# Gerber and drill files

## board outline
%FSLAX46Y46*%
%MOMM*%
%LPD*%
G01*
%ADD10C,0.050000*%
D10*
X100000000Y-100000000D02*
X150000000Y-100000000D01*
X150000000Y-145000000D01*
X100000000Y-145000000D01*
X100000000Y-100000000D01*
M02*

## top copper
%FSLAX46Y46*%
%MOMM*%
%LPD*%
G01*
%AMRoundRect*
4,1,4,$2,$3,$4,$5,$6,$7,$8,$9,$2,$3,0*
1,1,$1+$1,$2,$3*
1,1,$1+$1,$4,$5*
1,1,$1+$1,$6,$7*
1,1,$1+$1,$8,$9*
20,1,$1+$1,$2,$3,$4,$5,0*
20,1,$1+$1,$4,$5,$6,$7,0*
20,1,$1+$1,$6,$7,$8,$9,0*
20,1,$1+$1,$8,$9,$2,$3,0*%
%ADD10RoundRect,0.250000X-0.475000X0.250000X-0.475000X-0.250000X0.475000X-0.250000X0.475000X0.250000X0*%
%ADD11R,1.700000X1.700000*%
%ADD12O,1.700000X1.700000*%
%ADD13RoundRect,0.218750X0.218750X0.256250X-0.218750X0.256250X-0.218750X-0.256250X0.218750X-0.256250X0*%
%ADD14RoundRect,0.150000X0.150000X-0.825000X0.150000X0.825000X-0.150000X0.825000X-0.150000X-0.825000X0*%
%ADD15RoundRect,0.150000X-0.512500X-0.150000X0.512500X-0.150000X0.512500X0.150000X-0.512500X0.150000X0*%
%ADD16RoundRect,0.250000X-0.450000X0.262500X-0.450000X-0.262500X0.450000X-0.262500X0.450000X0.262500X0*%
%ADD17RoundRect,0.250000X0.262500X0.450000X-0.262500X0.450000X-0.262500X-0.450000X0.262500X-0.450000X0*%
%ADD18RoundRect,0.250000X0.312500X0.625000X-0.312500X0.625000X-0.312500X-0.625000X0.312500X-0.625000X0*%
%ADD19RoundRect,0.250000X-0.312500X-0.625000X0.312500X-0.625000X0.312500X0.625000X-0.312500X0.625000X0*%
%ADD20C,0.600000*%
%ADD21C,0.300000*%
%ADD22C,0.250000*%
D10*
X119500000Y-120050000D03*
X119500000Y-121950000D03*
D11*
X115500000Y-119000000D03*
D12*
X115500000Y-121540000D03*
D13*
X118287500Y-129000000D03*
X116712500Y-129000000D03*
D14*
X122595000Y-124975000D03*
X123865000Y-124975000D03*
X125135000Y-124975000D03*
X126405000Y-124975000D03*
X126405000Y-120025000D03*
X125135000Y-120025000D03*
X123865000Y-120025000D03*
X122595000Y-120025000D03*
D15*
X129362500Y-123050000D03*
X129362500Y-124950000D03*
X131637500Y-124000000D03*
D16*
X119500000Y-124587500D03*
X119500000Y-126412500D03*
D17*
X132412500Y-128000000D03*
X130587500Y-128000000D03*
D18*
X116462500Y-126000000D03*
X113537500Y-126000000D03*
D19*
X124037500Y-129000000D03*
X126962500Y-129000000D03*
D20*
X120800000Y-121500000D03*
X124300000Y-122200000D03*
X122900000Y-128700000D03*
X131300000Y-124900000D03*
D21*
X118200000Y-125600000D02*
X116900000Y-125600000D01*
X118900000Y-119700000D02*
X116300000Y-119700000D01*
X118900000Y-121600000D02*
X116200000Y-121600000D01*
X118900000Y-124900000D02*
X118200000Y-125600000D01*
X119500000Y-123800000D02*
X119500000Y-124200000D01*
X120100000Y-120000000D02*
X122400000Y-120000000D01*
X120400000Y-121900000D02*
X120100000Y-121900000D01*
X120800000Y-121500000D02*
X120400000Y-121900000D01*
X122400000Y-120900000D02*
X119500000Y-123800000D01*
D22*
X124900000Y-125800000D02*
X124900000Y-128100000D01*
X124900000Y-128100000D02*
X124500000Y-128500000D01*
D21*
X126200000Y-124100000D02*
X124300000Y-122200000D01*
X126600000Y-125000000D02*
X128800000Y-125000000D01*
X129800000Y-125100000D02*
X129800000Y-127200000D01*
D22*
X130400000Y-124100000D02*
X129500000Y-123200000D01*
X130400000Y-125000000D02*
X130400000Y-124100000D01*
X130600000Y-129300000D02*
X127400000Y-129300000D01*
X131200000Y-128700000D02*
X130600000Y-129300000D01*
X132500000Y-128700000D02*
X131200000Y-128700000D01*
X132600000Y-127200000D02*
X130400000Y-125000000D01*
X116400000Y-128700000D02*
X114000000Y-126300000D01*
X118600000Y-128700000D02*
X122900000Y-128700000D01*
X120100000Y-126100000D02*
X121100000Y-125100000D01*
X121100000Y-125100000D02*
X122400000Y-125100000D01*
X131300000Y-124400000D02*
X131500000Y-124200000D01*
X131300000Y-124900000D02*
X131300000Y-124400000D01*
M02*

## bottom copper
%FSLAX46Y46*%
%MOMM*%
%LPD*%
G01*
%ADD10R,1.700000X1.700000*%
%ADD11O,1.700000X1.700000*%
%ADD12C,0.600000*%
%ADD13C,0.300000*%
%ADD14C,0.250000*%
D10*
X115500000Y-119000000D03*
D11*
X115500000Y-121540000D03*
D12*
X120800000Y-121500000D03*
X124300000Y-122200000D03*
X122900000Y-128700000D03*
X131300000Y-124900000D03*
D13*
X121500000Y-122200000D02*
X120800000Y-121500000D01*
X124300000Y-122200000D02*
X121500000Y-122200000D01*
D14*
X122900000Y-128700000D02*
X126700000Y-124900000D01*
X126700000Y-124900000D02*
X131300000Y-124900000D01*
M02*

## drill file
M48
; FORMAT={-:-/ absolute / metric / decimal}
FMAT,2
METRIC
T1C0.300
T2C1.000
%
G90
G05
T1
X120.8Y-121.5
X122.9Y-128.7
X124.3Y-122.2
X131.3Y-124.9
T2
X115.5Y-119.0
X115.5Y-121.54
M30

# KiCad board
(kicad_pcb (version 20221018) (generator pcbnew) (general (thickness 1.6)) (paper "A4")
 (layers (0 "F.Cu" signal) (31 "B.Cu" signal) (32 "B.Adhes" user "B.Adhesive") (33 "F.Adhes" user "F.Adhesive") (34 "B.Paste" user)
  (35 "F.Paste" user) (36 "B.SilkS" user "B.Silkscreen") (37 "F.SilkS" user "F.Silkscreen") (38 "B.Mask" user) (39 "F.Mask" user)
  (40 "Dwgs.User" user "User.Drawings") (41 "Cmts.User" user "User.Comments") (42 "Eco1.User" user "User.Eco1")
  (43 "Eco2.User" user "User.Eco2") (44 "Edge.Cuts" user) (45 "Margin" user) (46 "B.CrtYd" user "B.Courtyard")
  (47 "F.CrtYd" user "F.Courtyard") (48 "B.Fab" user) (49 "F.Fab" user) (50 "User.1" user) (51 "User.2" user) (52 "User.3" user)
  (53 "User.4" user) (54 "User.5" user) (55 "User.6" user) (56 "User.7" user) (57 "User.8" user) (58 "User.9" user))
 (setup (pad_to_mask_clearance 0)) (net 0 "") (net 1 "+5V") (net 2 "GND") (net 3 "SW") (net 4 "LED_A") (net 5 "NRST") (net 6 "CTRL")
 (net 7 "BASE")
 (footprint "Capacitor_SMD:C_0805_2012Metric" (layer "F.Cu") (at 119.5 121 -90)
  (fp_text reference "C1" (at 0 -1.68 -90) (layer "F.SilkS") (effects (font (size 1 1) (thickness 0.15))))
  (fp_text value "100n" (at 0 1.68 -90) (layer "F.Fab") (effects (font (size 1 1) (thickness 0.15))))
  (pad "1" smd roundrect (at -0.95 0 270) (size 1 1.45) (layers "F.Cu" "F.Paste" "F.Mask") (roundrect_rratio 0.25) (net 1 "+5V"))
  (pad "2" smd roundrect (at 0.95 0 270) (size 1 1.45) (layers "F.Cu" "F.Paste" "F.Mask") (roundrect_rratio 0.25) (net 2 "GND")))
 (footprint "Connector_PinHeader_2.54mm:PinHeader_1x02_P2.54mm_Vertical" (layer "F.Cu") (at 115.5 119)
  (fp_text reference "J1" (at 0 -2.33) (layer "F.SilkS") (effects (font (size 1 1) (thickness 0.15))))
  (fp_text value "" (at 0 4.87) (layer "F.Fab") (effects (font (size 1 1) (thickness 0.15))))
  (pad "1" thru_hole rect (at 0 0) (size 1.7 1.7) (drill 1) (layers "*.Cu" "*.Mask") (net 1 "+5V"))
  (pad "2" thru_hole oval (at 0 2.54) (size 1.7 1.7) (drill 1) (layers "*.Cu" "*.Mask") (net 2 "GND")))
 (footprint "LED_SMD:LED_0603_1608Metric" (layer "F.Cu") (at 117.5 129 180)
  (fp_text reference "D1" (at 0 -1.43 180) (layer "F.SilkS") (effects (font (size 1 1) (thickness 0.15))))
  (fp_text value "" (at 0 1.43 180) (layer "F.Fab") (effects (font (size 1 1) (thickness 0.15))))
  (pad "1" smd roundrect (at -0.7875 0 180) (size 0.875 0.95) (layers "F.Cu" "F.Paste" "F.Mask") (roundrect_rratio 0.25) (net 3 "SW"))
  (pad "2" smd roundrect (at 0.7875 0 180) (size 0.875 0.95) (layers "F.Cu" "F.Paste" "F.Mask") (roundrect_rratio 0.25) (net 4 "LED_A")))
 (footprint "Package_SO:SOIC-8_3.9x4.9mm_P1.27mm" (layer "F.Cu") (at 124.5 122.5 90)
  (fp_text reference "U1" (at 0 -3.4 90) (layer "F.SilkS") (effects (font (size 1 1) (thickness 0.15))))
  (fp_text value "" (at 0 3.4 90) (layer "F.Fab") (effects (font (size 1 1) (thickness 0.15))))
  (pad "1" smd roundrect (at -2.475 -1.905 90) (size 1.95 0.6) (layers "F.Cu" "F.Paste" "F.Mask") (roundrect_rratio 0.25) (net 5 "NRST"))
  (pad "2" smd roundrect (at -2.475 -0.635 90) (size 1.95 0.6) (layers "F.Cu" "F.Paste" "F.Mask") (roundrect_rratio 0.25))
  (pad "3" smd roundrect (at -2.475 0.635 90) (size 1.95 0.6) (layers "F.Cu" "F.Paste" "F.Mask") (roundrect_rratio 0.25) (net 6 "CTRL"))
  (pad "4" smd roundrect (at -2.475 1.905 90) (size 1.95 0.6) (layers "F.Cu" "F.Paste" "F.Mask") (roundrect_rratio 0.25) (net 2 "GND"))
  (pad "5" smd roundrect (at 2.475 1.905 90) (size 1.95 0.6) (layers "F.Cu" "F.Paste" "F.Mask") (roundrect_rratio 0.25))
  (pad "6" smd roundrect (at 2.475 0.635 90) (size 1.95 0.6) (layers "F.Cu" "F.Paste" "F.Mask") (roundrect_rratio 0.25))
  (pad "7" smd roundrect (at 2.475 -0.635 90) (size 1.95 0.6) (layers "F.Cu" "F.Paste" "F.Mask") (roundrect_rratio 0.25))
  (pad "8" smd roundrect (at 2.475 -1.905 90) (size 1.95 0.6) (layers "F.Cu" "F.Paste" "F.Mask") (roundrect_rratio 0.25) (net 1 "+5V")))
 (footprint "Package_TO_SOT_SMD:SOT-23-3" (layer "F.Cu") (at 130.5 124)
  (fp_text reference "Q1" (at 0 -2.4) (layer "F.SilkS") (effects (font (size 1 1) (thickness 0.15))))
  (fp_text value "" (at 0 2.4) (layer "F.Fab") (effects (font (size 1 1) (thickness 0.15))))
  (pad "1" smd roundrect (at -1.1375 -0.95) (size 1.325 0.6) (layers "F.Cu" "F.Paste" "F.Mask") (roundrect_rratio 0.25) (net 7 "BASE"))
  (pad "2" smd roundrect (at -1.1375 0.95) (size 1.325 0.6) (layers "F.Cu" "F.Paste" "F.Mask") (roundrect_rratio 0.25) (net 2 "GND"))
  (pad "3" smd roundrect (at 1.1375 0) (size 1.325 0.6) (layers "F.Cu" "F.Paste" "F.Mask") (roundrect_rratio 0.25) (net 3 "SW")))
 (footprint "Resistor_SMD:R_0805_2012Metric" (layer "F.Cu") (at 119.5 125.5 -90)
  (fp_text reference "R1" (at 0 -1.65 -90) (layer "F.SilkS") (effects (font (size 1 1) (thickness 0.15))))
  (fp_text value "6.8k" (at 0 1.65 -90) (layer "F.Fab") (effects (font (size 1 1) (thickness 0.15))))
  (pad "1" smd roundrect (at -0.9125 0 270) (size 1.025 1.4) (layers "F.Cu" "F.Paste" "F.Mask") (roundrect_rratio 0.243902) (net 1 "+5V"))
  (pad "2" smd roundrect (at 0.9125 0 270) (size 1.025 1.4) (layers "F.Cu" "F.Paste" "F.Mask") (roundrect_rratio 0.243902) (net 5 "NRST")))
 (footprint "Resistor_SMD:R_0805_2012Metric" (layer "F.Cu") (at 131.5 128 180)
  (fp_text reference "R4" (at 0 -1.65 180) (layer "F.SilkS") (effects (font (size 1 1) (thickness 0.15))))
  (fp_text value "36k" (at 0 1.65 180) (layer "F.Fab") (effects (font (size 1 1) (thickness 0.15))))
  (pad "1" smd roundrect (at -0.9125 0 180) (size 1.025 1.4) (layers "F.Cu" "F.Paste" "F.Mask") (roundrect_rratio 0.243902) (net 7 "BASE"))
  (pad "2" smd roundrect (at 0.9125 0 180) (size 1.025 1.4) (layers "F.Cu" "F.Paste" "F.Mask") (roundrect_rratio 0.243902) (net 2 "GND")))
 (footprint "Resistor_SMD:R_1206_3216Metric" (layer "F.Cu") (at 115 126 180)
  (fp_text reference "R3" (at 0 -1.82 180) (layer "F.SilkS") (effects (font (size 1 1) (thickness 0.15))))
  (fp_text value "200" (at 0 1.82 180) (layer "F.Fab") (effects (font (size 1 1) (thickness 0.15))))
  (pad "1" smd roundrect (at -1.4625 0 180) (size 1.125 1.75) (layers "F.Cu" "F.Paste" "F.Mask") (roundrect_rratio 0.222222) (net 1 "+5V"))
  (pad "2" smd roundrect (at 1.4625 0 180) (size 1.125 1.75) (layers "F.Cu" "F.Paste" "F.Mask") (roundrect_rratio 0.222222) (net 4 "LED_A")))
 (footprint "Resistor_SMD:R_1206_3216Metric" (layer "F.Cu") (at 125.5 129)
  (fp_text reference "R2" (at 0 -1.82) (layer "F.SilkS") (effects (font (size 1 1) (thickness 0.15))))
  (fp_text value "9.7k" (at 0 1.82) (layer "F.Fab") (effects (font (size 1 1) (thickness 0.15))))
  (pad "1" smd roundrect (at -1.4625 0) (size 1.125 1.75) (layers "F.Cu" "F.Paste" "F.Mask") (roundrect_rratio 0.222222) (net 6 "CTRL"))
  (pad "2" smd roundrect (at 1.4625 0) (size 1.125 1.75) (layers "F.Cu" "F.Paste" "F.Mask") (roundrect_rratio 0.222222) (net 7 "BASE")))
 (gr_rect (start 100 100) (end 150 145) (stroke (width 0.05) (type default)) (fill none) (layer "Edge.Cuts"))
 (segment (start 118.2 125.6) (end 116.9 125.6) (width 0.3) (layer "F.Cu") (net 1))
 (segment (start 118.9 119.7) (end 116.3 119.7) (width 0.3) (layer "F.Cu") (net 1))
 (segment (start 118.9 121.6) (end 116.2 121.6) (width 0.3) (layer "F.Cu") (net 2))
 (segment (start 118.9 124.9) (end 118.2 125.6) (width 0.3) (layer "F.Cu") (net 1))
 (segment (start 119.5 123.8) (end 119.5 124.2) (width 0.3) (layer "F.Cu") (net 1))
 (segment (start 120.1 120) (end 122.4 120) (width 0.3) (layer "F.Cu") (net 1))
 (segment (start 120.4 121.9) (end 120.1 121.9) (width 0.3) (layer "F.Cu") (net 2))
 (segment (start 120.8 121.5) (end 120.4 121.9) (width 0.3) (layer "F.Cu") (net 2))
 (segment (start 122.4 120.9) (end 119.5 123.8) (width 0.3) (layer "F.Cu") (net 1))
 (segment (start 124.9 125.8) (end 124.9 128.1) (width 0.25) (layer "F.Cu") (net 6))
 (segment (start 124.9 128.1) (end 124.5 128.5) (width 0.25) (layer "F.Cu") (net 6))
 (segment (start 126.2 124.1) (end 124.3 122.2) (width 0.3) (layer "F.Cu") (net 2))
 (segment (start 126.6 125) (end 128.8 125) (width 0.3) (layer "F.Cu") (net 2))
 (segment (start 129.8 125.1) (end 129.8 127.2) (width 0.3) (layer "F.Cu") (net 2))
 (segment (start 130.4 124.1) (end 129.5 123.2) (width 0.25) (layer "F.Cu") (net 7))
 (segment (start 130.4 125) (end 130.4 124.1) (width 0.25) (layer "F.Cu") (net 7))
 (segment (start 130.6 129.3) (end 127.4 129.3) (width 0.25) (layer "F.Cu") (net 7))
 (segment (start 131.2 128.7) (end 130.6 129.3) (width 0.25) (layer "F.Cu") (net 7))
 (segment (start 132.5 128.7) (end 131.2 128.7) (width 0.25) (layer "F.Cu") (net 7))
 (segment (start 132.6 127.2) (end 130.4 125) (width 0.25) (layer "F.Cu") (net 7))
 (via (at 120.8 121.5) (size 0.6) (drill 0.3) (layers "F.Cu" "B.Cu") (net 2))
 (via (at 124.3 122.2) (size 0.6) (drill 0.3) (layers "F.Cu" "B.Cu") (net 2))
 (segment (start 116.4 128.7) (end 114 126.3) (width 0.25) (layer "F.Cu") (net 4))
 (segment (start 118.6 128.7) (end 122.9 128.7) (width 0.25) (layer "F.Cu") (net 3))
 (segment (start 120.1 126.1) (end 121.1 125.1) (width 0.25) (layer "F.Cu") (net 5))
 (segment (start 121.1 125.1) (end 122.4 125.1) (width 0.25) (layer "F.Cu") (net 5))
 (segment (start 121.5 122.2) (end 120.8 121.5) (width 0.3) (layer "B.Cu") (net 2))
 (segment (start 124.3 122.2) (end 121.5 122.2) (width 0.3) (layer "B.Cu") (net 2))
 (segment (start 131.3 124.4) (end 131.5 124.2) (width 0.25) (layer "F.Cu") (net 3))
 (segment (start 131.3 124.9) (end 131.3 124.4) (width 0.25) (layer "F.Cu") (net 3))
 (via (at 122.9 128.7) (size 0.6) (drill 0.3) (layers "F.Cu" "B.Cu") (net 3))
 (via (at 131.3 124.9) (size 0.6) (drill 0.3) (layers "F.Cu" "B.Cu") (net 3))
 (segment (start 122.9 128.7) (end 126.7 124.9) (width 0.25) (layer "B.Cu") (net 3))
 (segment (start 126.7 124.9) (end 131.3 124.9) (width 0.25) (layer "B.Cu") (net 3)))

